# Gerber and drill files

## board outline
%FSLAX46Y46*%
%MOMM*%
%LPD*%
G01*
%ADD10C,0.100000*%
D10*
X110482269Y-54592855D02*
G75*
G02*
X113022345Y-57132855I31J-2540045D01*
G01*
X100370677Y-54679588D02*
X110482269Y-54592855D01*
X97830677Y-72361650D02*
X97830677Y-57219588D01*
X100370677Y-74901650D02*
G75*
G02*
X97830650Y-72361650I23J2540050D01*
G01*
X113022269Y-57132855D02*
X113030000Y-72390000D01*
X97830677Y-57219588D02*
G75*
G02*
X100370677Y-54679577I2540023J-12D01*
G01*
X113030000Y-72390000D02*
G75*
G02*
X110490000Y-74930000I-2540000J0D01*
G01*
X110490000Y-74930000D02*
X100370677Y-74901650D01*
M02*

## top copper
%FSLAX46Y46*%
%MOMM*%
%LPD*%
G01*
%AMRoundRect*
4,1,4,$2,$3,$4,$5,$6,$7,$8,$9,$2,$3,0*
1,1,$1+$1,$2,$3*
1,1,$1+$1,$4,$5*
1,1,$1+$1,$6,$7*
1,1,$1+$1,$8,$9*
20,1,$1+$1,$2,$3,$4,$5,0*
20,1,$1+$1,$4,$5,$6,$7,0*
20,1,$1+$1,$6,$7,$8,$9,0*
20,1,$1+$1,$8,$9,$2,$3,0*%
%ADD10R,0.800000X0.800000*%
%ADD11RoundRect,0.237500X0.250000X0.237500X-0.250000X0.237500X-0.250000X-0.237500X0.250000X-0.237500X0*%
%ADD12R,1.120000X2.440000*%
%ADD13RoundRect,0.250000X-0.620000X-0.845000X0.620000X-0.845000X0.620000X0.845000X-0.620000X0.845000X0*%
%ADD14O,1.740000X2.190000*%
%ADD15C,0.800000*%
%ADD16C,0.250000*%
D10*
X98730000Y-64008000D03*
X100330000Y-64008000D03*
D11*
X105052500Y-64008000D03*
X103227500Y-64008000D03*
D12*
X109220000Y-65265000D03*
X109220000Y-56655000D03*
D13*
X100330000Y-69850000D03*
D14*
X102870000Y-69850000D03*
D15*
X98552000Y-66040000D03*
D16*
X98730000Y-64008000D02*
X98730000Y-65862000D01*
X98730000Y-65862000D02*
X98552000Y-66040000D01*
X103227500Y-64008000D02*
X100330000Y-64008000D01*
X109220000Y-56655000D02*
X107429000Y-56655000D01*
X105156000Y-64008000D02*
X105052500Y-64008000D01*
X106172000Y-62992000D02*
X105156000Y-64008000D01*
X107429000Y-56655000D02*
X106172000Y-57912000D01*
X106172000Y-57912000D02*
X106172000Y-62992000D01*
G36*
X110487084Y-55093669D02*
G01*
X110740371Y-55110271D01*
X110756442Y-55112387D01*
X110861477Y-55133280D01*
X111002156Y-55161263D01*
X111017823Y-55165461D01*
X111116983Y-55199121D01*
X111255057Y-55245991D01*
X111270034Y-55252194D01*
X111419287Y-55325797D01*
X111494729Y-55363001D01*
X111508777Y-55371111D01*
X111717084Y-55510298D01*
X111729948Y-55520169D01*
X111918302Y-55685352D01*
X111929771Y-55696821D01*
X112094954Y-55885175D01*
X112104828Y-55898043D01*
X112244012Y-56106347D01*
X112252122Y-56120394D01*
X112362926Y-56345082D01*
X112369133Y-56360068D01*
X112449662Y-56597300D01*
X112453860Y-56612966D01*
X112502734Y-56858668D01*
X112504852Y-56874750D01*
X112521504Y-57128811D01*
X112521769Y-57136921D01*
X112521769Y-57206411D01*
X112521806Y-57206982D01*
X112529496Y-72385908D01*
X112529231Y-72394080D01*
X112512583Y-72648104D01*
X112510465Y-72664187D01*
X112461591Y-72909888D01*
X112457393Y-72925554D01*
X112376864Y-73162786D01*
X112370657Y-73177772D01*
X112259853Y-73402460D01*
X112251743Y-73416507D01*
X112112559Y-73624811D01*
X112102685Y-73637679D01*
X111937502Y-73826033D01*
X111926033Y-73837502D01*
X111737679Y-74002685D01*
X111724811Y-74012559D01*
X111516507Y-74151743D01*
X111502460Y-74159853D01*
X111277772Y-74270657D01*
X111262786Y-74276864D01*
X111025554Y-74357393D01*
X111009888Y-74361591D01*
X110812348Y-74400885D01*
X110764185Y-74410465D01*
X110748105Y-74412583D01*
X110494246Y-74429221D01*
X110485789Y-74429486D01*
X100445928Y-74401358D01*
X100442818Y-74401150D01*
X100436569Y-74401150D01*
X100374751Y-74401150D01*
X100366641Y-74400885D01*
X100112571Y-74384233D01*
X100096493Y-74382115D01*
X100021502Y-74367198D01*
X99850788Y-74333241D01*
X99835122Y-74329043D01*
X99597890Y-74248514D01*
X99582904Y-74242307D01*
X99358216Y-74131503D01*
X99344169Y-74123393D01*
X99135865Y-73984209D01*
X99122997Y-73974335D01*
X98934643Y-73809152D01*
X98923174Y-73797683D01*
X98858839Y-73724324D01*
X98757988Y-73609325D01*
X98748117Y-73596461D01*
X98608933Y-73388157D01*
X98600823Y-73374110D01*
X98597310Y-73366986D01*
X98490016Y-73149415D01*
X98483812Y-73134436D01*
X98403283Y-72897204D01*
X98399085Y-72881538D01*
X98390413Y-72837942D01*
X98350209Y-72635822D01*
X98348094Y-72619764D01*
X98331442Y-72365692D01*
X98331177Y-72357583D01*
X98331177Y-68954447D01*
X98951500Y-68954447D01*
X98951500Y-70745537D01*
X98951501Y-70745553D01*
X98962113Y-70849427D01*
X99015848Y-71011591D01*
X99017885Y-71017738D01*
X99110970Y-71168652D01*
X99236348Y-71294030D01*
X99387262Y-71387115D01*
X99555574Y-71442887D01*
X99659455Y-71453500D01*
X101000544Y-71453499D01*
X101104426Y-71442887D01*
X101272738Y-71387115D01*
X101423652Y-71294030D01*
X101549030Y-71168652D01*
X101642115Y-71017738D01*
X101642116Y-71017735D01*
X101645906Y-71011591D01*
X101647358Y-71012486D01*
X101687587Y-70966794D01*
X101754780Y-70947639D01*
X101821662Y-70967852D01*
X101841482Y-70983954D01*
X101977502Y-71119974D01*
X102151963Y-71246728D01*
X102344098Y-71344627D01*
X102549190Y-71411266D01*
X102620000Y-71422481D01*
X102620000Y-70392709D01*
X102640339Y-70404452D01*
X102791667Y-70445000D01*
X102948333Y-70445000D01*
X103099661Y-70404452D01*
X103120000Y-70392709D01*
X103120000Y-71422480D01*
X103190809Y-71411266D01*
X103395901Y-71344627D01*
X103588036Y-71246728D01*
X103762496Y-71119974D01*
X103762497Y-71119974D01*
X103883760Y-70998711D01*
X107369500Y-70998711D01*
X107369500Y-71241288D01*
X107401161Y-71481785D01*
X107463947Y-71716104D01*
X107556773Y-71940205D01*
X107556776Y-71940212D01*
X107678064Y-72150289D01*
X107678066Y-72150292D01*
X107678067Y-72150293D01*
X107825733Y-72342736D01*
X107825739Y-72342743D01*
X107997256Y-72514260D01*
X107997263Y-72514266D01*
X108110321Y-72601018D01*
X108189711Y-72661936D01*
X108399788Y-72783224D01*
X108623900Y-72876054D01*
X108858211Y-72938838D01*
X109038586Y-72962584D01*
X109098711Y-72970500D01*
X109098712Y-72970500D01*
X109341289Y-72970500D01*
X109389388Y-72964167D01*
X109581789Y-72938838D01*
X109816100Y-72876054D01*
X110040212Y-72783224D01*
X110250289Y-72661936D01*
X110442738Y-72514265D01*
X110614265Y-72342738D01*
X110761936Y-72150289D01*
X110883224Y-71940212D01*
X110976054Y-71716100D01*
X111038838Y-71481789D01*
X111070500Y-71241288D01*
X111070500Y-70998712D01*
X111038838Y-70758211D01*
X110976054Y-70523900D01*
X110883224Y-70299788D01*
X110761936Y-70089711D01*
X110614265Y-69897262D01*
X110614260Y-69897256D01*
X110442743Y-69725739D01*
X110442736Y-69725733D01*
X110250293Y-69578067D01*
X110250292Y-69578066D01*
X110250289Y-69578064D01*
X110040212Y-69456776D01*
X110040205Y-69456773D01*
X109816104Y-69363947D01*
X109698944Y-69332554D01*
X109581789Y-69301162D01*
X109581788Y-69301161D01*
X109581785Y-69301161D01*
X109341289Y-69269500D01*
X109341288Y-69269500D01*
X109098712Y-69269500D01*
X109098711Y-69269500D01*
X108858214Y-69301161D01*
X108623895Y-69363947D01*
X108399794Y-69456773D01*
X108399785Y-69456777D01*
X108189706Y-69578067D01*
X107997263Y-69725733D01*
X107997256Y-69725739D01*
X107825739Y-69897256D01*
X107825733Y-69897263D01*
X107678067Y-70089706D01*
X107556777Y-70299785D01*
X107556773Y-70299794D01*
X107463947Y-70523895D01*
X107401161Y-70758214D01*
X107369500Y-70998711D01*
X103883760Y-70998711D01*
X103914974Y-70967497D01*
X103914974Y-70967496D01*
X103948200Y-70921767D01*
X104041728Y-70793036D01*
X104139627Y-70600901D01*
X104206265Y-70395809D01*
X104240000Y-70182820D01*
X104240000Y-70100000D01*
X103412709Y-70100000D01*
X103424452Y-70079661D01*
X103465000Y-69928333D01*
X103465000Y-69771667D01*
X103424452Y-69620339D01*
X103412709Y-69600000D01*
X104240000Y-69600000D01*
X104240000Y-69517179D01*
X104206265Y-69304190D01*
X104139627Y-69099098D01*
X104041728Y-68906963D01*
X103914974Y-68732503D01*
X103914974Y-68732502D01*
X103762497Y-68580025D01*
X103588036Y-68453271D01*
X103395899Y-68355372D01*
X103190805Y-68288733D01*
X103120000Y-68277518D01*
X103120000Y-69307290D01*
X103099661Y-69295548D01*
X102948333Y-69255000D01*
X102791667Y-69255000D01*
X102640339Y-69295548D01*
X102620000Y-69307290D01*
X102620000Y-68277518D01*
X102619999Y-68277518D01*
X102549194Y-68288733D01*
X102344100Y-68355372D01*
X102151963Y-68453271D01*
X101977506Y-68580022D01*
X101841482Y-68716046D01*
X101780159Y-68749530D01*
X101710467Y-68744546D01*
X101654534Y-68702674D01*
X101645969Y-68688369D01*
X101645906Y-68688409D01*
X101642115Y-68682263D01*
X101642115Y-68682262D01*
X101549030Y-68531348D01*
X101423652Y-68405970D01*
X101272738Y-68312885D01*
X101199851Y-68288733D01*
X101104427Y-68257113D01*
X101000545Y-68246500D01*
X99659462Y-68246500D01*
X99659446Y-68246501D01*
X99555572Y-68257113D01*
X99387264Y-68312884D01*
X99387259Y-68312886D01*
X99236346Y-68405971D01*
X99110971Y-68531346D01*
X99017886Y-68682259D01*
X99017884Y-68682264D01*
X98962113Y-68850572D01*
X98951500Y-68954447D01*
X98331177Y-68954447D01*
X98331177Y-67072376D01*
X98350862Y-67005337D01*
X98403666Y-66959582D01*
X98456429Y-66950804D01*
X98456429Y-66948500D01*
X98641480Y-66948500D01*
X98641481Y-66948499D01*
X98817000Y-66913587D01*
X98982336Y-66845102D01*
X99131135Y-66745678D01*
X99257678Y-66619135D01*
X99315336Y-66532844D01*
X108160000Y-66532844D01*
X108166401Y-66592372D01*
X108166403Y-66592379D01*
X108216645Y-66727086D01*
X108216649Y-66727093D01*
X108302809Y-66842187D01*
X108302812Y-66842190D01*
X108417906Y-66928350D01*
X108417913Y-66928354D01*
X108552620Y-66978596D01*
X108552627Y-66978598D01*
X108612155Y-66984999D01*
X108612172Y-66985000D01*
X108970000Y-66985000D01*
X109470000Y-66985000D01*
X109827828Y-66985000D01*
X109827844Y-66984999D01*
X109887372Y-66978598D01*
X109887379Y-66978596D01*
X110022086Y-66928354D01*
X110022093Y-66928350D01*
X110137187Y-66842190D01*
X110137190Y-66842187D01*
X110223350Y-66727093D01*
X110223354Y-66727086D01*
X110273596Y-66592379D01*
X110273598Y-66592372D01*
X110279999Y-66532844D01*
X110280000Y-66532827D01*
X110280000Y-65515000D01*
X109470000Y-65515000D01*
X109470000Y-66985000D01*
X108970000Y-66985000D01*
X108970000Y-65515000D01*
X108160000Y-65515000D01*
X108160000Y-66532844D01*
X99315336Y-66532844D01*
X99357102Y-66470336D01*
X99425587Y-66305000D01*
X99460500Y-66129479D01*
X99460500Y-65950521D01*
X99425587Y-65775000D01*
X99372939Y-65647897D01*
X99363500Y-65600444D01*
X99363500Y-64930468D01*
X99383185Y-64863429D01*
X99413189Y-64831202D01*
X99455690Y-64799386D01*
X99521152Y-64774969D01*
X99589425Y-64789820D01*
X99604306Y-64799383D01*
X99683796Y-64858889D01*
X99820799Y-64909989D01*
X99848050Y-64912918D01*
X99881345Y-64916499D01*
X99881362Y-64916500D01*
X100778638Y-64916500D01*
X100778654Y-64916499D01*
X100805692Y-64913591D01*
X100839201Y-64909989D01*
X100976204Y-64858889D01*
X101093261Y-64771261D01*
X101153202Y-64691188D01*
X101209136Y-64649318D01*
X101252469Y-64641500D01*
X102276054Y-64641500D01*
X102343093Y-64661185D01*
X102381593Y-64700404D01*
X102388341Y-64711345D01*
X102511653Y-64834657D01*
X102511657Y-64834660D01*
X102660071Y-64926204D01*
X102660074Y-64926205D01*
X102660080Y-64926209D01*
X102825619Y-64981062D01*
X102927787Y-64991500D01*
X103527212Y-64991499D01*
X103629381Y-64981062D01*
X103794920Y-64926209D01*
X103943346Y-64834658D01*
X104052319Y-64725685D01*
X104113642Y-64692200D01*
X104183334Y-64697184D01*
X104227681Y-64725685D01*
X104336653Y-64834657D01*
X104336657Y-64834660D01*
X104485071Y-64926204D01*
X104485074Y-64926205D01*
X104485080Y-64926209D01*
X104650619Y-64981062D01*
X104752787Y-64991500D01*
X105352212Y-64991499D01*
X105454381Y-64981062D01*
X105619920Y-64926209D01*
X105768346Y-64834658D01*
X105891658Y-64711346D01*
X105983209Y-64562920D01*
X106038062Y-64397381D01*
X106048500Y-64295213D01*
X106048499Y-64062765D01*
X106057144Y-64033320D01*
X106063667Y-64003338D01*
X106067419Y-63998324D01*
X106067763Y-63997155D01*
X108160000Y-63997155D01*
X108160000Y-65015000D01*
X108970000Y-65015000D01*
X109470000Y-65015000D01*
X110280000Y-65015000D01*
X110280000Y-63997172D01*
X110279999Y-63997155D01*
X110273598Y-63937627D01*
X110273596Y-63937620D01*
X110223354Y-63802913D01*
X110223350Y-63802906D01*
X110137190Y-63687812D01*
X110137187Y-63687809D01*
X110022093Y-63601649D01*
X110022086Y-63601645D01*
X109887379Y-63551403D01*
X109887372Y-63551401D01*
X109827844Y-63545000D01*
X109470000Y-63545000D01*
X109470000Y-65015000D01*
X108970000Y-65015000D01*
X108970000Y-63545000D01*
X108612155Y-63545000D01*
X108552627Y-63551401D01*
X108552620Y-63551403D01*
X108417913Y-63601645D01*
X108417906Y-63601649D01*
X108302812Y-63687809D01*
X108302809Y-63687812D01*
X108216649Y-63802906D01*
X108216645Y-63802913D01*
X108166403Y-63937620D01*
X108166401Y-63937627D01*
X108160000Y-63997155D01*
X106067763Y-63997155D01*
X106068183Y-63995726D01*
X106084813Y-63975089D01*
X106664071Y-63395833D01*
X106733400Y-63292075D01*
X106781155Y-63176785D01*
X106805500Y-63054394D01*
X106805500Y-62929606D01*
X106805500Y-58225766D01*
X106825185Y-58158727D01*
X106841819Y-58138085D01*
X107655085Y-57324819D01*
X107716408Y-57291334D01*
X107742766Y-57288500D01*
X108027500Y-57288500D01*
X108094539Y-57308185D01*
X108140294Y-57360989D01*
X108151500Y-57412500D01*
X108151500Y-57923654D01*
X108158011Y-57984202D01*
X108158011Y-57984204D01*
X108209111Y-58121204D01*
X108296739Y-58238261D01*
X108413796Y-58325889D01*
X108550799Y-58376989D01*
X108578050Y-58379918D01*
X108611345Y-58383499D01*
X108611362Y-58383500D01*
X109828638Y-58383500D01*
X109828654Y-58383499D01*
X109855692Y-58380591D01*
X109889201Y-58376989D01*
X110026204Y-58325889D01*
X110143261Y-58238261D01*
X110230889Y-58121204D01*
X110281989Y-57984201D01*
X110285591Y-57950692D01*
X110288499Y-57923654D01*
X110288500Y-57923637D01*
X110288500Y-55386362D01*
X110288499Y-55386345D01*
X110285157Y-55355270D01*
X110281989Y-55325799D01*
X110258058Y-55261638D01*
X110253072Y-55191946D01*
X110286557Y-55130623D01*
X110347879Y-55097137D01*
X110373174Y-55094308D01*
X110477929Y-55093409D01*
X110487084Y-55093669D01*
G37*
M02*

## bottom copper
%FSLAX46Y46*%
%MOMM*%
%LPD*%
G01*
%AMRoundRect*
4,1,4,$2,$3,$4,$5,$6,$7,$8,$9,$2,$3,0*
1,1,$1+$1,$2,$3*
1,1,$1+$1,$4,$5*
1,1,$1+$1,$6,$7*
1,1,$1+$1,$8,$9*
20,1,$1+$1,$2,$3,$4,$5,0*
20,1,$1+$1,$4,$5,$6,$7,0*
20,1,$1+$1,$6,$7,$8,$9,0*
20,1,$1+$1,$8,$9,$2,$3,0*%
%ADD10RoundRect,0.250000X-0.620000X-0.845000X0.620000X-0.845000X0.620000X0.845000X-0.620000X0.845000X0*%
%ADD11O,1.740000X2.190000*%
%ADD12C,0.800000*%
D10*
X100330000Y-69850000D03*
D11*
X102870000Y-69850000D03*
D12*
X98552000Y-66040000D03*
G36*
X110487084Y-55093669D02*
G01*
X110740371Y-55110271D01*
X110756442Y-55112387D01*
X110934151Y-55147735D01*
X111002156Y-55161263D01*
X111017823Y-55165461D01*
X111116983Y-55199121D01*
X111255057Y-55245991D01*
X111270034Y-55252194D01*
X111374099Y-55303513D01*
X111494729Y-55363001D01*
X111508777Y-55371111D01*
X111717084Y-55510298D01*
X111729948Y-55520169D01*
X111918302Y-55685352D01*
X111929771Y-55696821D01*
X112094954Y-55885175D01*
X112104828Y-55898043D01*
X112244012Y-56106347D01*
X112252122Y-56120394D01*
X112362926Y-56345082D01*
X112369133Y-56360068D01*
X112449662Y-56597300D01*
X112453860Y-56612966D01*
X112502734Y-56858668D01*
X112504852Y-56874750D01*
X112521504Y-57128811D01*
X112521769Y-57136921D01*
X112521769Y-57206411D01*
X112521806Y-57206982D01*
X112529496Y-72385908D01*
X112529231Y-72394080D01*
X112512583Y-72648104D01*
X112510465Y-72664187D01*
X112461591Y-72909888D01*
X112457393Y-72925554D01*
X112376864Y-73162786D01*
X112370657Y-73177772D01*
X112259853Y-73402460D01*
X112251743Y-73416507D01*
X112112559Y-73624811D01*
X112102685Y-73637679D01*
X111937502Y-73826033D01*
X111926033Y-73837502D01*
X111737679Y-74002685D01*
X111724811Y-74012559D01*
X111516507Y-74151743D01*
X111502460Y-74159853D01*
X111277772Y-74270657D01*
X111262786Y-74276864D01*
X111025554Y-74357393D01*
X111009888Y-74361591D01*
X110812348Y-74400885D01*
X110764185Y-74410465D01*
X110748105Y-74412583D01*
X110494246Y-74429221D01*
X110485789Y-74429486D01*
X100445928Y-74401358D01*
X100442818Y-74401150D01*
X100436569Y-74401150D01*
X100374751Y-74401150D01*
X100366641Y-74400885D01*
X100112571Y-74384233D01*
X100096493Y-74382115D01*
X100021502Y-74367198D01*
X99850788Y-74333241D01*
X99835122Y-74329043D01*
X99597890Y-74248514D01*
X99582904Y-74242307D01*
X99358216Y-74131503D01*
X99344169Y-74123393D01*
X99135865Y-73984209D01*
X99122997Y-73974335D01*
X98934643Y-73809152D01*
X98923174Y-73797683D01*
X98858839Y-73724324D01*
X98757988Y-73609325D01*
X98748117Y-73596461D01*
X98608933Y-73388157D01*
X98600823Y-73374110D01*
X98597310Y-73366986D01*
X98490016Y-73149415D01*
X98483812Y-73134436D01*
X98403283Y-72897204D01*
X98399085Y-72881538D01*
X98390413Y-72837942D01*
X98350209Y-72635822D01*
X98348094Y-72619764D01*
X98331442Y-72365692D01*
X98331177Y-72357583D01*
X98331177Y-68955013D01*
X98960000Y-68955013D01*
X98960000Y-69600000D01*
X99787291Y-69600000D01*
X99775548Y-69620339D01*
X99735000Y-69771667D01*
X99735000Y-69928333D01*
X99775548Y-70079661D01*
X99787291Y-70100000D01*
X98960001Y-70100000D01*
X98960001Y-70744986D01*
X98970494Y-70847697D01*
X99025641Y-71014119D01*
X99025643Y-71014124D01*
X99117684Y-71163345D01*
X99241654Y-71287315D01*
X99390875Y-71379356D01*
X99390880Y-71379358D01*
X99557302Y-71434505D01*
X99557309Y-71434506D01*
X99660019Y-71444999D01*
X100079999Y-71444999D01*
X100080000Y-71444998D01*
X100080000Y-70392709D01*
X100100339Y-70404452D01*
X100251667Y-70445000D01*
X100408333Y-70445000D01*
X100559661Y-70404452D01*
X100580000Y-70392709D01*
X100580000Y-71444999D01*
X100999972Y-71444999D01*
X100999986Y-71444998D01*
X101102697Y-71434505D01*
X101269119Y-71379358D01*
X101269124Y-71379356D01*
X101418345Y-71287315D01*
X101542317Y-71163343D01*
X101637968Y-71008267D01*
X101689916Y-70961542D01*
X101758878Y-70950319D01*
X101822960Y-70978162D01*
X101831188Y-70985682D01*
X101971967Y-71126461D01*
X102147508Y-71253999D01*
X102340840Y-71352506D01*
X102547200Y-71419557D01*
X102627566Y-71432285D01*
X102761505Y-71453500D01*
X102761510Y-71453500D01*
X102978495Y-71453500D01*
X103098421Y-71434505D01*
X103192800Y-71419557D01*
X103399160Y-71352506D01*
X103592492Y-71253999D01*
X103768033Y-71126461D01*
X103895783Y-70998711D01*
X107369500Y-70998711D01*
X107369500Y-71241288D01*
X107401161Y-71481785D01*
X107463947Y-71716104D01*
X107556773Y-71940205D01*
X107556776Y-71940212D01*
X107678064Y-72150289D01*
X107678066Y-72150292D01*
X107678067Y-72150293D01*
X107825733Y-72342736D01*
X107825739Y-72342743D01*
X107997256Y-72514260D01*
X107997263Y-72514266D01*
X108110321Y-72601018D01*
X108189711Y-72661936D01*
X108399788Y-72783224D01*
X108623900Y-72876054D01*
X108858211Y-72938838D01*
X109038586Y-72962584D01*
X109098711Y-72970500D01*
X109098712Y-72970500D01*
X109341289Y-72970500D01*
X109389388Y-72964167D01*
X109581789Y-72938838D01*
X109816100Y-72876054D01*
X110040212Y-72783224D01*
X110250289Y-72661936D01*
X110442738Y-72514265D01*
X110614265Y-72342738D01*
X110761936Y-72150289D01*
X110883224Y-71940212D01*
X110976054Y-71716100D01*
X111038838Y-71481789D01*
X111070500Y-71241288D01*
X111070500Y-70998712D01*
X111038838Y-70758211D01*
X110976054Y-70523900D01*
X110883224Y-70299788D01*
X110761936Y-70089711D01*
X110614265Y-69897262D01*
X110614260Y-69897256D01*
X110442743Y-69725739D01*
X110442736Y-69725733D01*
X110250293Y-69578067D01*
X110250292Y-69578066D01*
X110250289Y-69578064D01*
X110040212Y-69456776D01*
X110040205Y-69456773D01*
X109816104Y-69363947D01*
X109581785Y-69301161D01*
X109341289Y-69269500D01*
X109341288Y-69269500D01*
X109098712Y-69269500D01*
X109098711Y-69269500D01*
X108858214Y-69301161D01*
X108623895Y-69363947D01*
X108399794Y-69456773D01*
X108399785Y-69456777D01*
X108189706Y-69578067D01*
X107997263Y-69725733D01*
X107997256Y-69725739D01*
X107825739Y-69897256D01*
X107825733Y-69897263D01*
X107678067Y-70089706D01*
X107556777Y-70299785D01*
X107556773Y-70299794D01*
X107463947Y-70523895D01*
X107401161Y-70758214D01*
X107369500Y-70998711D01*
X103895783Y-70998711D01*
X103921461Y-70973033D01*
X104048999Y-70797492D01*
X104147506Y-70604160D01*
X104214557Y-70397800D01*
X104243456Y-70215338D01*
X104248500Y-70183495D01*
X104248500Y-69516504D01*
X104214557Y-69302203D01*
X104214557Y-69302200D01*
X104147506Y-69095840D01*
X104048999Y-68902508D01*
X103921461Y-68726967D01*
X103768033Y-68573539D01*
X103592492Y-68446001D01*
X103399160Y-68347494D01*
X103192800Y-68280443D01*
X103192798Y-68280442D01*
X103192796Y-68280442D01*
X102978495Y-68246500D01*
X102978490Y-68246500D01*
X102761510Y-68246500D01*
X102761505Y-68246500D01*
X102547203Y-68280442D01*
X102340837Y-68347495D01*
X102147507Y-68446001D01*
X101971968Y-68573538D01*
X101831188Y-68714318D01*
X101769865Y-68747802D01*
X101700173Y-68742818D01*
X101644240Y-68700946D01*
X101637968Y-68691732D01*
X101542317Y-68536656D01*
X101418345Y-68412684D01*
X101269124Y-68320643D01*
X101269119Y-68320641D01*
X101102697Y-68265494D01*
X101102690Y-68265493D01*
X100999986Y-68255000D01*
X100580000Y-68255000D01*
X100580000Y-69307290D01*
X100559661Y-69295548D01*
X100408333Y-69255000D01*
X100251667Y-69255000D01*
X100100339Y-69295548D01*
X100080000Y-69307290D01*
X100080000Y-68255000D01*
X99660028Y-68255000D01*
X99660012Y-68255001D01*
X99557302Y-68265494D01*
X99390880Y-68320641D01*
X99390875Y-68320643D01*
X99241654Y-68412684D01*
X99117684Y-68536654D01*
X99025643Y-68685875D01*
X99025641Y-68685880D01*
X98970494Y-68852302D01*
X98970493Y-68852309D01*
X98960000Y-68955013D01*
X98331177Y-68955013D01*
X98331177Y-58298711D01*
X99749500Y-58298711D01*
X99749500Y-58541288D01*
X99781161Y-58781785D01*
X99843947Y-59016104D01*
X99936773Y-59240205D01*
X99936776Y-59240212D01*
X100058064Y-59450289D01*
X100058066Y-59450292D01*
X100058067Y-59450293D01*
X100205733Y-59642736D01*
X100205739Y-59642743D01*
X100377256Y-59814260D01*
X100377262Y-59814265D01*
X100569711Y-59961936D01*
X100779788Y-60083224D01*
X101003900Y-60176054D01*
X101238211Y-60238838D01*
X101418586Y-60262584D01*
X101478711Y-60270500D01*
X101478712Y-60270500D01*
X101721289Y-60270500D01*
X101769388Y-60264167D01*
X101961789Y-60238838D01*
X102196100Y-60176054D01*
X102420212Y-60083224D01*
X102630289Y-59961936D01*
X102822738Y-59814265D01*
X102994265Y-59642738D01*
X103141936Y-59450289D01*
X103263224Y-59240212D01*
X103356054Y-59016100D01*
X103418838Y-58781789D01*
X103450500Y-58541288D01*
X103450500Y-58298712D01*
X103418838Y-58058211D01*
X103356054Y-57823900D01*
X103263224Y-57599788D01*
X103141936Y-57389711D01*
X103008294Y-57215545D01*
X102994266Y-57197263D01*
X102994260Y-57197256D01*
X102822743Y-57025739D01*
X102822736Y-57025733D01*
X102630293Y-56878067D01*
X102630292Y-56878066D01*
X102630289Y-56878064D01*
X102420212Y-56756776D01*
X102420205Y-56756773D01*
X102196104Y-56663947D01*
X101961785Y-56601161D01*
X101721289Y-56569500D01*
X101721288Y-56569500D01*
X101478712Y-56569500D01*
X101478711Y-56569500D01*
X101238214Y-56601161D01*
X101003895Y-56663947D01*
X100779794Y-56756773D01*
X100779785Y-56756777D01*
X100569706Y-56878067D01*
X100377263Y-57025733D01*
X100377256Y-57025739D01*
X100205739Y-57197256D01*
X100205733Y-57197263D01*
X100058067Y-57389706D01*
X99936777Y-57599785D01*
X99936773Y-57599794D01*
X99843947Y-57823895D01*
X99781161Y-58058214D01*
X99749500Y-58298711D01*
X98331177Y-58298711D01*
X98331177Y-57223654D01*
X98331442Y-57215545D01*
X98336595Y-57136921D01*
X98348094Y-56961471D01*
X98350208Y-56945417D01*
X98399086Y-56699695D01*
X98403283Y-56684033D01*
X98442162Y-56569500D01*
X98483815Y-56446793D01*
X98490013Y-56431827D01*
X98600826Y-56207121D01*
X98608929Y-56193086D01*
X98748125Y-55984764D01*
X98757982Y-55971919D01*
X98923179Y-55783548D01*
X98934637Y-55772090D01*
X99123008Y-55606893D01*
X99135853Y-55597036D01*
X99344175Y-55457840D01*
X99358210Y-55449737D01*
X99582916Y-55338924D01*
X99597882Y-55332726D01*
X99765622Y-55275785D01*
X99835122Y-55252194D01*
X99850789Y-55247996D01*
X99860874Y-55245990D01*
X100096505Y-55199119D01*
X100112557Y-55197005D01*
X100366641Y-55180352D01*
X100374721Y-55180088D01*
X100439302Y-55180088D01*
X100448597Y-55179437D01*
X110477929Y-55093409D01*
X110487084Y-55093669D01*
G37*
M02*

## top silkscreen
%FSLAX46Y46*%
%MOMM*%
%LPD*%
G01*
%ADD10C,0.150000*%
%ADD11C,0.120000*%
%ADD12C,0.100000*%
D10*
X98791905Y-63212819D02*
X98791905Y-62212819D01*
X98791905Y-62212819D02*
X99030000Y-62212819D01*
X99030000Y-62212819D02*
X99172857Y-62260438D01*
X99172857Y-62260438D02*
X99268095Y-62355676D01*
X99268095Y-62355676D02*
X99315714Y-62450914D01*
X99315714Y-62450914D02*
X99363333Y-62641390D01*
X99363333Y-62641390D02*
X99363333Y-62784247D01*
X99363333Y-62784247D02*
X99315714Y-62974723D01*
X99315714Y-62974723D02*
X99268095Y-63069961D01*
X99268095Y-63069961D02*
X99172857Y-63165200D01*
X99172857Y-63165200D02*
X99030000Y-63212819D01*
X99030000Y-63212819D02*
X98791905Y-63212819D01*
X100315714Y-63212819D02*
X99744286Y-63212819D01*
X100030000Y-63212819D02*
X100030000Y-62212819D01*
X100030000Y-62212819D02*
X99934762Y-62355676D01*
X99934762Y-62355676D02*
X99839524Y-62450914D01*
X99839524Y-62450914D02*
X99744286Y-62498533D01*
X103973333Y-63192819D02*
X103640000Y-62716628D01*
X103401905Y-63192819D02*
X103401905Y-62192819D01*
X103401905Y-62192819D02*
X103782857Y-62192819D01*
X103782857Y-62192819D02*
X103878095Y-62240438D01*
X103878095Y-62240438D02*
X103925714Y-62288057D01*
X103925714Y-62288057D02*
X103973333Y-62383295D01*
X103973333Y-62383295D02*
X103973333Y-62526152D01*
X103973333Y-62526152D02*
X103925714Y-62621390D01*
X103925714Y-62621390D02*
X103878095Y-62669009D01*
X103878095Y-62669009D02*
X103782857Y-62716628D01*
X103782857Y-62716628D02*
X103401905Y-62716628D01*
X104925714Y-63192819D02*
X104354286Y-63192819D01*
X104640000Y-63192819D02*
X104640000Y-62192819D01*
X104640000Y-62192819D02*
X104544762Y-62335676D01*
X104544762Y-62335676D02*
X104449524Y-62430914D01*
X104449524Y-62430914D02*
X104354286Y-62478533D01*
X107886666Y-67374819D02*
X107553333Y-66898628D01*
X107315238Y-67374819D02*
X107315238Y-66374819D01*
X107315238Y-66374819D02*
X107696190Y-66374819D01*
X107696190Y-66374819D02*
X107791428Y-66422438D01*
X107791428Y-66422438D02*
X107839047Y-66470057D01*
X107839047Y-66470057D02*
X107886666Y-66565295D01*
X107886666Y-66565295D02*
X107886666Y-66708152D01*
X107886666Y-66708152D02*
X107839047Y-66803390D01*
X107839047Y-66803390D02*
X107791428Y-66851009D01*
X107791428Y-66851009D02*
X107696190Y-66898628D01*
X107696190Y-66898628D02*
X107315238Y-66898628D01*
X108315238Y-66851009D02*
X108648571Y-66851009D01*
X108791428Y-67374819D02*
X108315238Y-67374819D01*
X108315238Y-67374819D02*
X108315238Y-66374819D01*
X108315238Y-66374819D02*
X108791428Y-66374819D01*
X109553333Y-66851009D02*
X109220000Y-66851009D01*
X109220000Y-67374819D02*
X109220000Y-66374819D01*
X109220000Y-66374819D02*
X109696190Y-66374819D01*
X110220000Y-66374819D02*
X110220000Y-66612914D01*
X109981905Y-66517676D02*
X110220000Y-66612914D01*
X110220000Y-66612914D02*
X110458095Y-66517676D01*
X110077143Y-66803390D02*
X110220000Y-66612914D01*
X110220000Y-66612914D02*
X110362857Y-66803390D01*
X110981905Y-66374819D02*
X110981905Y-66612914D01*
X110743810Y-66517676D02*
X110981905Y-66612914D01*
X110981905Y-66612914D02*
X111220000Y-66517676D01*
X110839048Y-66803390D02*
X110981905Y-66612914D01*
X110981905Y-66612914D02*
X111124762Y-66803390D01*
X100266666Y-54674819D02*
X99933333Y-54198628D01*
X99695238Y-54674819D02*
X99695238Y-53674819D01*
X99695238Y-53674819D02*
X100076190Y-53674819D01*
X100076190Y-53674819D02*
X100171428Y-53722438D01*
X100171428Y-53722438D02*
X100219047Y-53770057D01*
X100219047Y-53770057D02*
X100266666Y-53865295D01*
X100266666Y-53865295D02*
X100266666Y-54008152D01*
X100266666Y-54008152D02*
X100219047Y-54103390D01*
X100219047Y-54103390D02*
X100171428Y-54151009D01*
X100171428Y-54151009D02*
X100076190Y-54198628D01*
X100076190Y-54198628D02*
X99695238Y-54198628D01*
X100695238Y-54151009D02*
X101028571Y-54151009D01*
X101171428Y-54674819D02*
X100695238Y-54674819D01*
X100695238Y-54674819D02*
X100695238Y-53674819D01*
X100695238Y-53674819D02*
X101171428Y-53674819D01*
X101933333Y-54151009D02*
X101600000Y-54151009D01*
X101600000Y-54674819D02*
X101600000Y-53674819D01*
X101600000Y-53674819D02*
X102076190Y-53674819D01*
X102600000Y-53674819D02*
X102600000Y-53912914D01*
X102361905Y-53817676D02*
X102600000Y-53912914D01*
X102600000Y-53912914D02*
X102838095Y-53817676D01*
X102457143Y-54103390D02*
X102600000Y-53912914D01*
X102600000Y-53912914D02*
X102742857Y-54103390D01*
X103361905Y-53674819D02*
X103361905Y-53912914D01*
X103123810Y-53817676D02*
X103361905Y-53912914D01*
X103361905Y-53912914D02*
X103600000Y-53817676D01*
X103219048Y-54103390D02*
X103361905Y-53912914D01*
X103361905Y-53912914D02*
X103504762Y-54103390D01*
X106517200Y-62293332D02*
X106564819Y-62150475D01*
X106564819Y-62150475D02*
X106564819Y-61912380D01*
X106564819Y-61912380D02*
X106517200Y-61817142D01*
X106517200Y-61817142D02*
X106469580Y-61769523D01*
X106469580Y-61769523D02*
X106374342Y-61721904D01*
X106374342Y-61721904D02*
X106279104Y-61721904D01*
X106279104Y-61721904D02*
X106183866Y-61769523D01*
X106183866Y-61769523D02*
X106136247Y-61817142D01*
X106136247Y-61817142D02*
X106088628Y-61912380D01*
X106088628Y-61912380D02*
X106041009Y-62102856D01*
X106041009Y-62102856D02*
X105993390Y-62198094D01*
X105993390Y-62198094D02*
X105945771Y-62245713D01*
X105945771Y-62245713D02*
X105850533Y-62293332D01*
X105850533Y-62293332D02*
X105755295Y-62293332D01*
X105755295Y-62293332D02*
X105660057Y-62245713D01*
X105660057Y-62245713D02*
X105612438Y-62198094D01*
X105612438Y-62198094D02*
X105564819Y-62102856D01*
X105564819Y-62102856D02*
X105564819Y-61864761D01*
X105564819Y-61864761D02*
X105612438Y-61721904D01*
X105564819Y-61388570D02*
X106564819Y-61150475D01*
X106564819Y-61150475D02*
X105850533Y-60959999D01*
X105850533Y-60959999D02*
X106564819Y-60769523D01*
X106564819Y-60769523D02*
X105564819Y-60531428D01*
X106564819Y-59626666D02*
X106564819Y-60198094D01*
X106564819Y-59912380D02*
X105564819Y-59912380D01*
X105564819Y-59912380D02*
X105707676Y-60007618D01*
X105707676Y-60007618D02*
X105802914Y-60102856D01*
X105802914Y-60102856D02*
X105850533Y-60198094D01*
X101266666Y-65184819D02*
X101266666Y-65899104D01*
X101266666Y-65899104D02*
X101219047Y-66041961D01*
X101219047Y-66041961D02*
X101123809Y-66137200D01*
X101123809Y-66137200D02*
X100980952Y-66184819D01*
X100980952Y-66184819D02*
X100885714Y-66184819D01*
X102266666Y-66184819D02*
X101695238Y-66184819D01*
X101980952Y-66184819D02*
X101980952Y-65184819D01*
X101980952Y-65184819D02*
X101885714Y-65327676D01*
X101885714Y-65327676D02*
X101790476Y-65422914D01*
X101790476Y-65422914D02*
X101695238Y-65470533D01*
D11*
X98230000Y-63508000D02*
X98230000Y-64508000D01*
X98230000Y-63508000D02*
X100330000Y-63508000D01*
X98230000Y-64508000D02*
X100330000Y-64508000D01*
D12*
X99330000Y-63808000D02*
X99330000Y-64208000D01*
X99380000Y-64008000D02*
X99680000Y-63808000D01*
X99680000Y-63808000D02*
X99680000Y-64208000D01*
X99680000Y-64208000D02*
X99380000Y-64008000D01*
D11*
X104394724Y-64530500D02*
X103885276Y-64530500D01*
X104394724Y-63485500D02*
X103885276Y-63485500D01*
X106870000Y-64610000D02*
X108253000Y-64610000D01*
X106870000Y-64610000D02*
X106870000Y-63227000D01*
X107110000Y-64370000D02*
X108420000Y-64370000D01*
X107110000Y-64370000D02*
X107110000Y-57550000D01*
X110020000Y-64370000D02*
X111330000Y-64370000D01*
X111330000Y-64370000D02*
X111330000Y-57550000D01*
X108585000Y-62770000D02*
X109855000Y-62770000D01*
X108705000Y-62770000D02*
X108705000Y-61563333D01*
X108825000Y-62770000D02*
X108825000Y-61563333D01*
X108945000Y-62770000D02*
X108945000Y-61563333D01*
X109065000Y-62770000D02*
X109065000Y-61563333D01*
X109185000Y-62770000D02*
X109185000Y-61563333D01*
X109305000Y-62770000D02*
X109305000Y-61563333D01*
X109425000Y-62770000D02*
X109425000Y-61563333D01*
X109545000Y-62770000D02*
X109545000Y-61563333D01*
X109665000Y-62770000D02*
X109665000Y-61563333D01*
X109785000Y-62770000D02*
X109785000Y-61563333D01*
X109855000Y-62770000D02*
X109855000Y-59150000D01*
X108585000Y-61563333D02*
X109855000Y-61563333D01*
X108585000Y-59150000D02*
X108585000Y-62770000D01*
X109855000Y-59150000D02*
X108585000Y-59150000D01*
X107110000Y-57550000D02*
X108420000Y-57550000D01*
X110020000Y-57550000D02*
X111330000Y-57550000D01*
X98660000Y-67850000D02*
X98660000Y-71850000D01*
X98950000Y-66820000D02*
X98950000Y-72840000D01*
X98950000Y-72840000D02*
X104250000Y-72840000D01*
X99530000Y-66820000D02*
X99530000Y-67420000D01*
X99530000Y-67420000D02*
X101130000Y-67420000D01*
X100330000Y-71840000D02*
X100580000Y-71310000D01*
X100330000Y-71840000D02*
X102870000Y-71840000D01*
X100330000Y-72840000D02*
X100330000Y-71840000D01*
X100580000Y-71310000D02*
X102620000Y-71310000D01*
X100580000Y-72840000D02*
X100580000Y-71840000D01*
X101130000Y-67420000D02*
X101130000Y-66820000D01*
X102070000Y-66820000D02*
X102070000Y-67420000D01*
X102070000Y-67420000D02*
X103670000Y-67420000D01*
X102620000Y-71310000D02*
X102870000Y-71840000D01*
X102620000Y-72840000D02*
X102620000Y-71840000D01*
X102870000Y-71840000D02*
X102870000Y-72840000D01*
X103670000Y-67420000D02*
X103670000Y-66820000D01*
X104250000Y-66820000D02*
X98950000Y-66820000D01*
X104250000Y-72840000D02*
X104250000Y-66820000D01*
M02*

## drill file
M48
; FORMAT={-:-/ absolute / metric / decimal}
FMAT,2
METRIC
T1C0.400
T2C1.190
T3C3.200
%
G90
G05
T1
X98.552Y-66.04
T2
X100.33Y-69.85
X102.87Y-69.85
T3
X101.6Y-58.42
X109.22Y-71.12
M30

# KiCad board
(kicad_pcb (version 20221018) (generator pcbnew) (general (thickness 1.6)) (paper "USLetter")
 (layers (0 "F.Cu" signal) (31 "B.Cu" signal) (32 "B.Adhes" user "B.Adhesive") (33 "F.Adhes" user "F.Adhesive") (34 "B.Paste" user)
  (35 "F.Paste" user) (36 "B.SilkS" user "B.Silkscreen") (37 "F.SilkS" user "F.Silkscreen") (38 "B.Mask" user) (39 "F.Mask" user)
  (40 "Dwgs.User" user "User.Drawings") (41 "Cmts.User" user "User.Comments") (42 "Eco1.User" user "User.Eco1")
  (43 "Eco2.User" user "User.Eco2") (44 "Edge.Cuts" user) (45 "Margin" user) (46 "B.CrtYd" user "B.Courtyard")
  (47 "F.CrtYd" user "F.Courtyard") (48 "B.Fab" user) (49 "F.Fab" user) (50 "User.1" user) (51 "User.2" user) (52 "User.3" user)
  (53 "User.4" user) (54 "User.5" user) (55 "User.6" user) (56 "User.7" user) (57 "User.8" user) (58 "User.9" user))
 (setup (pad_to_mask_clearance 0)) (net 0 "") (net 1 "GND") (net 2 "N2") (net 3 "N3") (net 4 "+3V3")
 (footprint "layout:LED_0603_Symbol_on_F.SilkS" (layer "F.Cu") (at 99.53 64.008)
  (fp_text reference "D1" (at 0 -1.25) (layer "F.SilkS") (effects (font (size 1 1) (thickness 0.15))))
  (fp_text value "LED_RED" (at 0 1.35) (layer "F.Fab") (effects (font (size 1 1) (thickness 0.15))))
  (fp_line (start -1.3 -0.5) (end -1.3 0.5) (stroke (width 0.12) (type solid)) (layer "F.SilkS"))
  (fp_line (start -1.3 -0.5) (end 0.8 -0.5) (stroke (width 0.12) (type solid)) (layer "F.SilkS"))
  (fp_line (start -1.3 0.5) (end 0.8 0.5) (stroke (width 0.12) (type solid)) (layer "F.SilkS"))
  (fp_line (start -0.2 -0.2) (end -0.2 0.2) (stroke (width 0.1) (type solid)) (layer "F.SilkS"))
  (fp_line (start -0.15 0) (end 0.15 -0.2) (stroke (width 0.1) (type solid)) (layer "F.SilkS"))
  (fp_line (start 0.15 -0.2) (end 0.15 0.2) (stroke (width 0.1) (type solid)) (layer "F.SilkS"))
  (fp_line (start 0.15 0.2) (end -0.15 0) (stroke (width 0.1) (type solid)) (layer "F.SilkS"))
  (pad "1" smd rect (at -0.8 0 180) (size 0.8 0.8) (layers "F.Cu" "F.Paste" "F.Mask") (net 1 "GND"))
  (pad "2" smd rect (at 0.8 0 180) (size 0.8 0.8) (layers "F.Cu" "F.Paste" "F.Mask") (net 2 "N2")))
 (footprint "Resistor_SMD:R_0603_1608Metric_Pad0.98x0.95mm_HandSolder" (layer "F.Cu") (at 104.14 64.008 180)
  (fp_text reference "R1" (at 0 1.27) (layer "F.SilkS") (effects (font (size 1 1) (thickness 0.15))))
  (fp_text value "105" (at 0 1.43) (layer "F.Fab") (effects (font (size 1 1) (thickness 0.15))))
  (fp_line (start -0.254724 -0.5225) (end 0.254724 -0.5225) (stroke (width 0.12) (type solid)) (layer "F.SilkS"))
  (fp_line (start -0.254724 0.5225) (end 0.254724 0.5225) (stroke (width 0.12) (type solid)) (layer "F.SilkS"))
  (pad "1" smd roundrect (at -0.9125 0 180) (size 0.975 0.95) (layers "F.Cu" "F.Paste" "F.Mask") (roundrect_rratio 0.25) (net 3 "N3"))
  (pad "2" smd roundrect (at 0.9125 0 180) (size 0.975 0.95) (layers "F.Cu" "F.Paste" "F.Mask") (roundrect_rratio 0.25) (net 2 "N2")))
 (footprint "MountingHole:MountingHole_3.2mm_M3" (layer "F.Cu") (at 109.22 71.12)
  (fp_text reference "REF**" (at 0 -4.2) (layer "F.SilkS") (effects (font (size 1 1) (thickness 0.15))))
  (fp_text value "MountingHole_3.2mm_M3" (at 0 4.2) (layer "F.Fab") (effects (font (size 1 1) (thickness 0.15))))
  (pad "" np_thru_hole circle (at 0 0) (size 3.2 3.2) (drill 3.2) (layers "*.Cu" "*.Mask")))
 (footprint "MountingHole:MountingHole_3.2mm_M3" (layer "F.Cu") (at 101.6 58.42)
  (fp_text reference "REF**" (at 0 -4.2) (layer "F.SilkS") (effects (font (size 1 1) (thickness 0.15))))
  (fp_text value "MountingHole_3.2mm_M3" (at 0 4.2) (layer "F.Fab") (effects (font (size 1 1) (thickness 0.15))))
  (pad "" np_thru_hole circle (at 0 0) (size 3.2 3.2) (drill 3.2) (layers "*.Cu" "*.Mask")))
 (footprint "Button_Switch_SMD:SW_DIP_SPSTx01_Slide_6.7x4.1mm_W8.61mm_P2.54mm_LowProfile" (layer "F.Cu") (at 109.22 60.96 90)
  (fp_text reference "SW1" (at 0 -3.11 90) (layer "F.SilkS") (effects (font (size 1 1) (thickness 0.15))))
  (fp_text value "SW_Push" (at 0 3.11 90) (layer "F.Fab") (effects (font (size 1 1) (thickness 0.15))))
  (fp_line (start -3.65 -2.35) (end -3.65 -0.967) (stroke (width 0.12) (type solid)) (layer "F.SilkS"))
  (fp_line (start -3.65 -2.35) (end -2.267 -2.35) (stroke (width 0.12) (type solid)) (layer "F.SilkS"))
  (fp_line (start -3.41 -2.11) (end -3.41 -0.8) (stroke (width 0.12) (type solid)) (layer "F.SilkS"))
  (fp_line (start -3.41 -2.11) (end 3.41 -2.11) (stroke (width 0.12) (type solid)) (layer "F.SilkS"))
  (fp_line (start -3.41 0.8) (end -3.41 2.11) (stroke (width 0.12) (type solid)) (layer "F.SilkS"))
  (fp_line (start -3.41 2.11) (end 3.41 2.11) (stroke (width 0.12) (type solid)) (layer "F.SilkS"))
  (fp_line (start -1.81 -0.635) (end -1.81 0.635) (stroke (width 0.12) (type solid)) (layer "F.SilkS"))
  (fp_line (start -1.81 -0.515) (end -0.603333 -0.515) (stroke (width 0.12) (type solid)) (layer "F.SilkS"))
  (fp_line (start -1.81 -0.395) (end -0.603333 -0.395) (stroke (width 0.12) (type solid)) (layer "F.SilkS"))
  (fp_line (start -1.81 -0.275) (end -0.603333 -0.275) (stroke (width 0.12) (type solid)) (layer "F.SilkS"))
  (fp_line (start -1.81 -0.155) (end -0.603333 -0.155) (stroke (width 0.12) (type solid)) (layer "F.SilkS"))
  (fp_line (start -1.81 -0.035) (end -0.603333 -0.035) (stroke (width 0.12) (type solid)) (layer "F.SilkS"))
  (fp_line (start -1.81 0.085) (end -0.603333 0.085) (stroke (width 0.12) (type solid)) (layer "F.SilkS"))
  (fp_line (start -1.81 0.205) (end -0.603333 0.205) (stroke (width 0.12) (type solid)) (layer "F.SilkS"))
  (fp_line (start -1.81 0.325) (end -0.603333 0.325) (stroke (width 0.12) (type solid)) (layer "F.SilkS"))
  (fp_line (start -1.81 0.445) (end -0.603333 0.445) (stroke (width 0.12) (type solid)) (layer "F.SilkS"))
  (fp_line (start -1.81 0.565) (end -0.603333 0.565) (stroke (width 0.12) (type solid)) (layer "F.SilkS"))
  (fp_line (start -1.81 0.635) (end 1.81 0.635) (stroke (width 0.12) (type solid)) (layer "F.SilkS"))
  (fp_line (start -0.603333 -0.635) (end -0.603333 0.635) (stroke (width 0.12) (type solid)) (layer "F.SilkS"))
  (fp_line (start 1.81 -0.635) (end -1.81 -0.635) (stroke (width 0.12) (type solid)) (layer "F.SilkS"))
  (fp_line (start 1.81 0.635) (end 1.81 -0.635) (stroke (width 0.12) (type solid)) (layer "F.SilkS"))
  (fp_line (start 3.41 -2.11) (end 3.41 -0.8) (stroke (width 0.12) (type solid)) (layer "F.SilkS"))
  (fp_line (start 3.41 0.8) (end 3.41 2.11) (stroke (width 0.12) (type solid)) (layer "F.SilkS"))
  (pad "1" smd rect (at -4.305 0 90) (size 2.44 1.12) (layers "F.Cu" "F.Paste" "F.Mask") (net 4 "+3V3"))
  (pad "2" smd rect (at 4.305 0 90) (size 2.44 1.12) (layers "F.Cu" "F.Paste" "F.Mask") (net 3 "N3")))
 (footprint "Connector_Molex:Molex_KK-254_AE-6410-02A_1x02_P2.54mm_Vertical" (layer "F.Cu") (at 100.33 69.85)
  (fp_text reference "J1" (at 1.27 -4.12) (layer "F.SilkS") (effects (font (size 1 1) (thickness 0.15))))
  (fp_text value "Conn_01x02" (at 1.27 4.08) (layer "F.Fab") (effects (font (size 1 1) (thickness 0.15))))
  (fp_line (start -1.67 -2) (end -1.67 2) (stroke (width 0.12) (type solid)) (layer "F.SilkS"))
  (fp_line (start -1.38 -3.03) (end -1.38 2.99) (stroke (width 0.12) (type solid)) (layer "F.SilkS"))
  (fp_line (start -1.38 2.99) (end 3.92 2.99) (stroke (width 0.12) (type solid)) (layer "F.SilkS"))
  (fp_line (start -0.8 -3.03) (end -0.8 -2.43) (stroke (width 0.12) (type solid)) (layer "F.SilkS"))
  (fp_line (start -0.8 -2.43) (end 0.8 -2.43) (stroke (width 0.12) (type solid)) (layer "F.SilkS"))
  (fp_line (start 0 1.99) (end 0.25 1.46) (stroke (width 0.12) (type solid)) (layer "F.SilkS"))
  (fp_line (start 0 1.99) (end 2.54 1.99) (stroke (width 0.12) (type solid)) (layer "F.SilkS"))
  (fp_line (start 0 2.99) (end 0 1.99) (stroke (width 0.12) (type solid)) (layer "F.SilkS"))
  (fp_line (start 0.25 1.46) (end 2.29 1.46) (stroke (width 0.12) (type solid)) (layer "F.SilkS"))
  (fp_line (start 0.25 2.99) (end 0.25 1.99) (stroke (width 0.12) (type solid)) (layer "F.SilkS"))
  (fp_line (start 0.8 -2.43) (end 0.8 -3.03) (stroke (width 0.12) (type solid)) (layer "F.SilkS"))
  (fp_line (start 1.74 -3.03) (end 1.74 -2.43) (stroke (width 0.12) (type solid)) (layer "F.SilkS"))
  (fp_line (start 1.74 -2.43) (end 3.34 -2.43) (stroke (width 0.12) (type solid)) (layer "F.SilkS"))
  (fp_line (start 2.29 1.46) (end 2.54 1.99) (stroke (width 0.12) (type solid)) (layer "F.SilkS"))
  (fp_line (start 2.29 2.99) (end 2.29 1.99) (stroke (width 0.12) (type solid)) (layer "F.SilkS"))
  (fp_line (start 2.54 1.99) (end 2.54 2.99) (stroke (width 0.12) (type solid)) (layer "F.SilkS"))
  (fp_line (start 3.34 -2.43) (end 3.34 -3.03) (stroke (width 0.12) (type solid)) (layer "F.SilkS"))
  (fp_line (start 3.92 -3.03) (end -1.38 -3.03) (stroke (width 0.12) (type solid)) (layer "F.SilkS"))
  (fp_line (start 3.92 2.99) (end 3.92 -3.03) (stroke (width 0.12) (type solid)) (layer "F.SilkS"))
  (pad "1" thru_hole roundrect (at 0 0) (size 1.74 2.19) (drill 1.19) (layers "*.Cu" "*.Mask") (roundrect_rratio 0.143678) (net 1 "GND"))
  (pad "2" thru_hole oval (at 2.54 0) (size 1.74 2.19) (drill 1.19) (layers "*.Cu" "*.Mask") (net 4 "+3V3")))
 (gr_arc (start 110.482269 54.592855) (mid 112.27832 55.336804) (end 113.022269 57.132855) (stroke (width 0.1) (type default))
  (layer "Edge.Cuts"))
 (gr_line (start 100.370677 54.679588) (end 110.482269 54.592855) (stroke (width 0.1) (type default)) (layer "Edge.Cuts"))
 (gr_line (start 97.830677 72.36165) (end 97.830677 57.219588) (stroke (width 0.1) (type default)) (layer "Edge.Cuts"))
 (gr_arc (start 100.370677 74.90165) (mid 98.574626 74.157701) (end 97.830677 72.36165) (stroke (width 0.1) (type default))
  (layer "Edge.Cuts"))
 (gr_line (start 113.022269 57.132855) (end 113.03 72.39) (stroke (width 0.1) (type default)) (layer "Edge.Cuts"))
 (gr_arc (start 97.830677 57.219588) (mid 98.574626 55.423537) (end 100.370677 54.679588) (stroke (width 0.1) (type default))
  (layer "Edge.Cuts"))
 (gr_arc (start 113.03 72.39) (mid 112.286051 74.186051) (end 110.49 74.93) (stroke (width 0.1) (type default)) (layer "Edge.Cuts"))
 (gr_line (start 110.49 74.93) (end 100.370677 74.90165) (stroke (width 0.1) (type default)) (layer "Edge.Cuts"))
 (segment (start 98.73 64.008) (end 98.73 65.862) (width 0.25) (layer "F.Cu") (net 1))
 (segment (start 98.73 65.862) (end 98.552 66.04) (width 0.25) (layer "F.Cu") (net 1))
 (via (at 98.552 66.04) (size 0.8) (drill 0.4) (layers "F.Cu" "B.Cu") (free) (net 1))
 (segment (start 103.2275 64.008) (end 100.33 64.008) (width 0.25) (layer "F.Cu") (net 2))
 (segment (start 109.22 56.655) (end 107.429 56.655) (width 0.25) (layer "F.Cu") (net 3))
 (segment (start 105.156 64.008) (end 105.0525 64.008) (width 0.25) (layer "F.Cu") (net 3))
 (segment (start 106.172 62.992) (end 105.156 64.008) (width 0.25) (layer "F.Cu") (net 3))
 (segment (start 107.429 56.655) (end 106.172 57.912) (width 0.25) (layer "F.Cu") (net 3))
 (segment (start 106.172 57.912) (end 106.172 62.992) (width 0.25) (layer "F.Cu") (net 3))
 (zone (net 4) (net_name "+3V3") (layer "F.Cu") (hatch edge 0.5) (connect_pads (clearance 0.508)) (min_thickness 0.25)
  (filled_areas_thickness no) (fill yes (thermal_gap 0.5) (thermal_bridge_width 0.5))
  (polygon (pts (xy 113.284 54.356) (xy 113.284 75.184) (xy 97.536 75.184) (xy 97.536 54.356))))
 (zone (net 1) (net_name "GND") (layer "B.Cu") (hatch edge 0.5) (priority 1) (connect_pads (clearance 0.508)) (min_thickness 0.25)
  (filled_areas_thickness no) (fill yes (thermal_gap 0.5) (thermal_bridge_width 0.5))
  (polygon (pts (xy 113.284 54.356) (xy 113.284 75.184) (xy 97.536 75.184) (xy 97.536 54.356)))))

